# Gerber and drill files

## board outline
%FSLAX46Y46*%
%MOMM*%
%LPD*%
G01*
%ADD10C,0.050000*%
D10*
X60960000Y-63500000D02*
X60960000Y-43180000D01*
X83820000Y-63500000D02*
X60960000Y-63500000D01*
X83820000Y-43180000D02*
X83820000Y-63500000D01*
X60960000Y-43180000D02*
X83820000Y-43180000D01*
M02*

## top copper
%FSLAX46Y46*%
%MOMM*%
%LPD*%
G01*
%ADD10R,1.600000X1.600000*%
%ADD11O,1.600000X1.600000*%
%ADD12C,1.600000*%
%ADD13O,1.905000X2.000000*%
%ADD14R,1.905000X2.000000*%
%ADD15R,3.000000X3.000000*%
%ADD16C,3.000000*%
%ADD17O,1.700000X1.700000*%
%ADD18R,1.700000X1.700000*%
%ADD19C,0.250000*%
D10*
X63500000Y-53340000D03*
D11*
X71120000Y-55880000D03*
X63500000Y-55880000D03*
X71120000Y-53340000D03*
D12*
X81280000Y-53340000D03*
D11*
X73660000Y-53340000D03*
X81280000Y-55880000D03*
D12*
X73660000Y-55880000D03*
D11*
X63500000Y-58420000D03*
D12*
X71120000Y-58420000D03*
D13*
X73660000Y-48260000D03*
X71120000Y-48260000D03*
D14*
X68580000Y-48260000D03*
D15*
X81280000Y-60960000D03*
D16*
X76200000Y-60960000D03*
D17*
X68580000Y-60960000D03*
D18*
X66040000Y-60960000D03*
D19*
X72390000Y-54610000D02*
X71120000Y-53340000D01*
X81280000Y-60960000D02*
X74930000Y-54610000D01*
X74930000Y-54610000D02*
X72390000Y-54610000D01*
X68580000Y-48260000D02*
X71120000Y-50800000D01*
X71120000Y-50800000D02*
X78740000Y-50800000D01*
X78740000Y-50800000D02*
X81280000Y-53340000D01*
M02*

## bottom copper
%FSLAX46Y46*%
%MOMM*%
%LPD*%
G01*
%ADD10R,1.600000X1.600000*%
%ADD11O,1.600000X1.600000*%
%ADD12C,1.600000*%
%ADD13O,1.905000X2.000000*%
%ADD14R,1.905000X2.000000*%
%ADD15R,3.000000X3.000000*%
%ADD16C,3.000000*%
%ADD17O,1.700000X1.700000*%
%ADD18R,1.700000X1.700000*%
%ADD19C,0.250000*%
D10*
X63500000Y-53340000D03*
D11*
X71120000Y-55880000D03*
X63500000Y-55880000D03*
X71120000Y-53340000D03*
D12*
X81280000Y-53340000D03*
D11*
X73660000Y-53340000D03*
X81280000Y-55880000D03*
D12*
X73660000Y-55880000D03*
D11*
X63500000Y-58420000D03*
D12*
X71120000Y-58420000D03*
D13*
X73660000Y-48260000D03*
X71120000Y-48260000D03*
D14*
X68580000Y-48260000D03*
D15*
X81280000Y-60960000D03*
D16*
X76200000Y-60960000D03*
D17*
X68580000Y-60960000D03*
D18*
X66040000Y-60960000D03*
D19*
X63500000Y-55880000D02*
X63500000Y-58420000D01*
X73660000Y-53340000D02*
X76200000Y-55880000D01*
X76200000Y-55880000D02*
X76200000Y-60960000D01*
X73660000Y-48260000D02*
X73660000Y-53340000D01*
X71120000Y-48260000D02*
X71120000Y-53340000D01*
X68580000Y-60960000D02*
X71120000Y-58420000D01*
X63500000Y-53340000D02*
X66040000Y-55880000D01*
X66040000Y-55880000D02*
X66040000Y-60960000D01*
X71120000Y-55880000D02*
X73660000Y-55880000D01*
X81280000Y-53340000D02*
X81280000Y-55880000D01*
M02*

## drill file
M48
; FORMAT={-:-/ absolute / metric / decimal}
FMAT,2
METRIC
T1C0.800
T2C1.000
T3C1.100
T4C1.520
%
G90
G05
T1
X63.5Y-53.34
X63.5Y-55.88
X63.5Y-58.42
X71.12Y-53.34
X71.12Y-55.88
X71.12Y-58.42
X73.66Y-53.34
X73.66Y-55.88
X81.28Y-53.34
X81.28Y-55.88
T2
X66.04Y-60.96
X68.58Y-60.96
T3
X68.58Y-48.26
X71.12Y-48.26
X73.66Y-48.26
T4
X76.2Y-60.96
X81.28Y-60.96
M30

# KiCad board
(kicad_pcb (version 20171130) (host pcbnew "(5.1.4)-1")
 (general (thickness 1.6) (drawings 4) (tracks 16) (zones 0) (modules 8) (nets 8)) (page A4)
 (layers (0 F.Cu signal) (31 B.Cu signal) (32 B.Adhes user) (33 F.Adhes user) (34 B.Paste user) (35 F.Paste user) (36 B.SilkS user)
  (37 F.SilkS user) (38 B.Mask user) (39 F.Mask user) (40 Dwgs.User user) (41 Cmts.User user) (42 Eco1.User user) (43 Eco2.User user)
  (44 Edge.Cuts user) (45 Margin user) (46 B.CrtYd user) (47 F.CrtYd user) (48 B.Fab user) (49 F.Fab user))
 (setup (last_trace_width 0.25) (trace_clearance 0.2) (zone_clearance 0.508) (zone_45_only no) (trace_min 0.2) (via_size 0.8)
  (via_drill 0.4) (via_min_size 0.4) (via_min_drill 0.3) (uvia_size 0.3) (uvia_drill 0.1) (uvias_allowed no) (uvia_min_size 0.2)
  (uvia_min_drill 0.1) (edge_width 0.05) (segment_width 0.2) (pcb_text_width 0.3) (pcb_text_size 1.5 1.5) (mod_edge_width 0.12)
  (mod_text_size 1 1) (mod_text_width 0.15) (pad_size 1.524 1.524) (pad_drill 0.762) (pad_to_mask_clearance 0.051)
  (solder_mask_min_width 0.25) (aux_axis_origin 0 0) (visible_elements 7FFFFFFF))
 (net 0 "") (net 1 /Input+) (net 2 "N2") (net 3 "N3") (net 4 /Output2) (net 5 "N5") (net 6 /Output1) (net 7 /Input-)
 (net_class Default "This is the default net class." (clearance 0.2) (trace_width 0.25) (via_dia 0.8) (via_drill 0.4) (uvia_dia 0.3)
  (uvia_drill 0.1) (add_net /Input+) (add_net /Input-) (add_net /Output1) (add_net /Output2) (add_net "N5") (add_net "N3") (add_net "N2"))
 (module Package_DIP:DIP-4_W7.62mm (layer F.Cu) (at 63.5 53.34)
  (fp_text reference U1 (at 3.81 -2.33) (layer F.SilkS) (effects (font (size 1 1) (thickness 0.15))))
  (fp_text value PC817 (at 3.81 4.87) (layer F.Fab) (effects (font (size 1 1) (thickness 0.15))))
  (pad 1 thru_hole rect (at 0 0) (size 1.6 1.6) (drill 0.8) (layers *.Cu *.Mask) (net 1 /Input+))
  (pad 3 thru_hole oval (at 7.62 2.54) (size 1.6 1.6) (drill 0.8) (layers *.Cu *.Mask) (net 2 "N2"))
  (pad 2 thru_hole oval (at 0 2.54) (size 1.6 1.6) (drill 0.8) (layers *.Cu *.Mask) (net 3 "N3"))
  (pad 4 thru_hole oval (at 7.62 0) (size 1.6 1.6) (drill 0.8) (layers *.Cu *.Mask) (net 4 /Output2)))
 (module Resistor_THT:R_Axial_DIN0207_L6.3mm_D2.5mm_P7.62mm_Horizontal (layer F.Cu) (at 81.28 53.34 180)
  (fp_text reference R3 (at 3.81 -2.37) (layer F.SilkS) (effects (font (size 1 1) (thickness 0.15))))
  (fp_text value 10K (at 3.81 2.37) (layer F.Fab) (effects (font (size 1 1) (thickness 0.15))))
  (pad 1 thru_hole circle (at 0 0 180) (size 1.6 1.6) (drill 0.8) (layers *.Cu *.Mask) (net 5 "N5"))
  (pad 2 thru_hole oval (at 7.62 0 180) (size 1.6 1.6) (drill 0.8) (layers *.Cu *.Mask) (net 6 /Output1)))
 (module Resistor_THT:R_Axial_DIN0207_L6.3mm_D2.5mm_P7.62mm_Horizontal (layer F.Cu) (at 73.66 55.88)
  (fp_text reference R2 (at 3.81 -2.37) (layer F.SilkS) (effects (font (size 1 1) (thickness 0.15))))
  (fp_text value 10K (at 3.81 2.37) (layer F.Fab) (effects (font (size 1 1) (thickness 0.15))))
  (pad 2 thru_hole oval (at 7.62 0) (size 1.6 1.6) (drill 0.8) (layers *.Cu *.Mask) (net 5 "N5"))
  (pad 1 thru_hole circle (at 0 0) (size 1.6 1.6) (drill 0.8) (layers *.Cu *.Mask) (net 2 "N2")))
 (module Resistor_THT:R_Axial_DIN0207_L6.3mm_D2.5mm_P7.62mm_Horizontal (layer F.Cu) (at 71.12 58.42 180)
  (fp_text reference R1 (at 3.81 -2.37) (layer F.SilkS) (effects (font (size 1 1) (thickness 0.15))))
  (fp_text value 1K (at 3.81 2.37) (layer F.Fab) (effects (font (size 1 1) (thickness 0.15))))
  (pad 2 thru_hole oval (at 7.62 0 180) (size 1.6 1.6) (drill 0.8) (layers *.Cu *.Mask) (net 3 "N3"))
  (pad 1 thru_hole circle (at 0 0 180) (size 1.6 1.6) (drill 0.8) (layers *.Cu *.Mask) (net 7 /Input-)))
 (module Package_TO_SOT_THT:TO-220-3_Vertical (layer F.Cu) (at 68.58 48.26)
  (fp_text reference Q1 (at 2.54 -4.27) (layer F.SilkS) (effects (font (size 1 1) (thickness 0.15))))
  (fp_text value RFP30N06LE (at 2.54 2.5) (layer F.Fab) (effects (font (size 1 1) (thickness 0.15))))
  (pad 3 thru_hole oval (at 5.08 0) (size 1.905 2) (drill 1.1) (layers *.Cu *.Mask) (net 6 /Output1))
  (pad 2 thru_hole oval (at 2.54 0) (size 1.905 2) (drill 1.1) (layers *.Cu *.Mask) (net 4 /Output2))
  (pad 1 thru_hole rect (at 0 0) (size 1.905 2) (drill 1.1) (layers *.Cu *.Mask) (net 5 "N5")))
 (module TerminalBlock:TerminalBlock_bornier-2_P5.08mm (layer F.Cu) (at 81.28 60.96 180)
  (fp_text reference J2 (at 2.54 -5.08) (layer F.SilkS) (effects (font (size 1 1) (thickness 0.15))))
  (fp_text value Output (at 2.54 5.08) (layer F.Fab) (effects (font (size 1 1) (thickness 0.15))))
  (pad 1 thru_hole rect (at 0 0 180) (size 3 3) (drill 1.52) (layers *.Cu *.Mask) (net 4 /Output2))
  (pad 2 thru_hole circle (at 5.08 0 180) (size 3 3) (drill 1.52) (layers *.Cu *.Mask) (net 6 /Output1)))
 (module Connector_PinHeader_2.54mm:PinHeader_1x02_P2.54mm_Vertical (layer F.Cu) (at 66.04 60.96 90)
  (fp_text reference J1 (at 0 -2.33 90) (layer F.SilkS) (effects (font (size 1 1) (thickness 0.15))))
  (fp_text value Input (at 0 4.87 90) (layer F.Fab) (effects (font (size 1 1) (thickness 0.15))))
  (pad 2 thru_hole oval (at 0 2.54 90) (size 1.7 1.7) (drill 1) (layers *.Cu *.Mask) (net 7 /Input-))
  (pad 1 thru_hole rect (at 0 0 90) (size 1.7 1.7) (drill 1) (layers *.Cu *.Mask) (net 1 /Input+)))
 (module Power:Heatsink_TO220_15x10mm (layer F.Cu) (at 71.12 44.45)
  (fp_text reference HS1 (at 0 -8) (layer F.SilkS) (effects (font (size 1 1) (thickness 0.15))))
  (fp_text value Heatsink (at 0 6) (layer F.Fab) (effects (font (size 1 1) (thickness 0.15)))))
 (gr_line (start 60.96 63.5) (end 60.96 43.18) (layer Edge.Cuts) (width 0.05))
 (gr_line (start 83.82 63.5) (end 60.96 63.5) (layer Edge.Cuts) (width 0.05))
 (gr_line (start 83.82 43.18) (end 83.82 63.5) (layer Edge.Cuts) (width 0.05))
 (gr_line (start 60.96 43.18) (end 83.82 43.18) (layer Edge.Cuts) (width 0.05))
 (segment (start 63.5 55.88) (end 63.5 58.42) (width 0.25) (layer B.Cu) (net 3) (status 30))
 (segment (start 73.66 53.34) (end 76.2 55.88) (width 0.25) (layer B.Cu) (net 6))
 (segment (start 76.2 55.88) (end 76.2 60.96) (width 0.25) (layer B.Cu) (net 6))
 (segment (start 73.66 48.26) (end 73.66 53.34) (width 0.25) (layer B.Cu) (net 6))
 (segment (start 72.39 54.61) (end 71.12 53.34) (width 0.25) (layer F.Cu) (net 4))
 (segment (start 71.12 48.26) (end 71.12 53.34) (width 0.25) (layer B.Cu) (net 4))
 (segment (start 81.28 60.96) (end 74.93 54.61) (width 0.25) (layer F.Cu) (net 4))
 (segment (start 74.93 54.61) (end 72.39 54.61) (width 0.25) (layer F.Cu) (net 4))
 (segment (start 68.58 60.96) (end 71.12 58.42) (width 0.25) (layer B.Cu) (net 7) (status 30))
 (segment (start 63.5 53.34) (end 66.04 55.88) (width 0.25) (layer B.Cu) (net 1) (status 10))
 (segment (start 66.04 55.88) (end 66.04 60.96) (width 0.25) (layer B.Cu) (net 1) (status 20))
 (segment (start 71.12 55.88) (end 73.66 55.88) (width 0.25) (layer B.Cu) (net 2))
 (segment (start 81.28 53.34) (end 81.28 55.88) (width 0.25) (layer B.Cu) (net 5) (status 30))
 (segment (start 68.58 48.26) (end 71.12 50.8) (width 0.25) (layer F.Cu) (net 5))
 (segment (start 71.12 50.8) (end 78.74 50.8) (width 0.25) (layer F.Cu) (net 5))
 (segment (start 78.74 50.8) (end 81.28 53.34) (width 0.25) (layer F.Cu) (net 5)))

